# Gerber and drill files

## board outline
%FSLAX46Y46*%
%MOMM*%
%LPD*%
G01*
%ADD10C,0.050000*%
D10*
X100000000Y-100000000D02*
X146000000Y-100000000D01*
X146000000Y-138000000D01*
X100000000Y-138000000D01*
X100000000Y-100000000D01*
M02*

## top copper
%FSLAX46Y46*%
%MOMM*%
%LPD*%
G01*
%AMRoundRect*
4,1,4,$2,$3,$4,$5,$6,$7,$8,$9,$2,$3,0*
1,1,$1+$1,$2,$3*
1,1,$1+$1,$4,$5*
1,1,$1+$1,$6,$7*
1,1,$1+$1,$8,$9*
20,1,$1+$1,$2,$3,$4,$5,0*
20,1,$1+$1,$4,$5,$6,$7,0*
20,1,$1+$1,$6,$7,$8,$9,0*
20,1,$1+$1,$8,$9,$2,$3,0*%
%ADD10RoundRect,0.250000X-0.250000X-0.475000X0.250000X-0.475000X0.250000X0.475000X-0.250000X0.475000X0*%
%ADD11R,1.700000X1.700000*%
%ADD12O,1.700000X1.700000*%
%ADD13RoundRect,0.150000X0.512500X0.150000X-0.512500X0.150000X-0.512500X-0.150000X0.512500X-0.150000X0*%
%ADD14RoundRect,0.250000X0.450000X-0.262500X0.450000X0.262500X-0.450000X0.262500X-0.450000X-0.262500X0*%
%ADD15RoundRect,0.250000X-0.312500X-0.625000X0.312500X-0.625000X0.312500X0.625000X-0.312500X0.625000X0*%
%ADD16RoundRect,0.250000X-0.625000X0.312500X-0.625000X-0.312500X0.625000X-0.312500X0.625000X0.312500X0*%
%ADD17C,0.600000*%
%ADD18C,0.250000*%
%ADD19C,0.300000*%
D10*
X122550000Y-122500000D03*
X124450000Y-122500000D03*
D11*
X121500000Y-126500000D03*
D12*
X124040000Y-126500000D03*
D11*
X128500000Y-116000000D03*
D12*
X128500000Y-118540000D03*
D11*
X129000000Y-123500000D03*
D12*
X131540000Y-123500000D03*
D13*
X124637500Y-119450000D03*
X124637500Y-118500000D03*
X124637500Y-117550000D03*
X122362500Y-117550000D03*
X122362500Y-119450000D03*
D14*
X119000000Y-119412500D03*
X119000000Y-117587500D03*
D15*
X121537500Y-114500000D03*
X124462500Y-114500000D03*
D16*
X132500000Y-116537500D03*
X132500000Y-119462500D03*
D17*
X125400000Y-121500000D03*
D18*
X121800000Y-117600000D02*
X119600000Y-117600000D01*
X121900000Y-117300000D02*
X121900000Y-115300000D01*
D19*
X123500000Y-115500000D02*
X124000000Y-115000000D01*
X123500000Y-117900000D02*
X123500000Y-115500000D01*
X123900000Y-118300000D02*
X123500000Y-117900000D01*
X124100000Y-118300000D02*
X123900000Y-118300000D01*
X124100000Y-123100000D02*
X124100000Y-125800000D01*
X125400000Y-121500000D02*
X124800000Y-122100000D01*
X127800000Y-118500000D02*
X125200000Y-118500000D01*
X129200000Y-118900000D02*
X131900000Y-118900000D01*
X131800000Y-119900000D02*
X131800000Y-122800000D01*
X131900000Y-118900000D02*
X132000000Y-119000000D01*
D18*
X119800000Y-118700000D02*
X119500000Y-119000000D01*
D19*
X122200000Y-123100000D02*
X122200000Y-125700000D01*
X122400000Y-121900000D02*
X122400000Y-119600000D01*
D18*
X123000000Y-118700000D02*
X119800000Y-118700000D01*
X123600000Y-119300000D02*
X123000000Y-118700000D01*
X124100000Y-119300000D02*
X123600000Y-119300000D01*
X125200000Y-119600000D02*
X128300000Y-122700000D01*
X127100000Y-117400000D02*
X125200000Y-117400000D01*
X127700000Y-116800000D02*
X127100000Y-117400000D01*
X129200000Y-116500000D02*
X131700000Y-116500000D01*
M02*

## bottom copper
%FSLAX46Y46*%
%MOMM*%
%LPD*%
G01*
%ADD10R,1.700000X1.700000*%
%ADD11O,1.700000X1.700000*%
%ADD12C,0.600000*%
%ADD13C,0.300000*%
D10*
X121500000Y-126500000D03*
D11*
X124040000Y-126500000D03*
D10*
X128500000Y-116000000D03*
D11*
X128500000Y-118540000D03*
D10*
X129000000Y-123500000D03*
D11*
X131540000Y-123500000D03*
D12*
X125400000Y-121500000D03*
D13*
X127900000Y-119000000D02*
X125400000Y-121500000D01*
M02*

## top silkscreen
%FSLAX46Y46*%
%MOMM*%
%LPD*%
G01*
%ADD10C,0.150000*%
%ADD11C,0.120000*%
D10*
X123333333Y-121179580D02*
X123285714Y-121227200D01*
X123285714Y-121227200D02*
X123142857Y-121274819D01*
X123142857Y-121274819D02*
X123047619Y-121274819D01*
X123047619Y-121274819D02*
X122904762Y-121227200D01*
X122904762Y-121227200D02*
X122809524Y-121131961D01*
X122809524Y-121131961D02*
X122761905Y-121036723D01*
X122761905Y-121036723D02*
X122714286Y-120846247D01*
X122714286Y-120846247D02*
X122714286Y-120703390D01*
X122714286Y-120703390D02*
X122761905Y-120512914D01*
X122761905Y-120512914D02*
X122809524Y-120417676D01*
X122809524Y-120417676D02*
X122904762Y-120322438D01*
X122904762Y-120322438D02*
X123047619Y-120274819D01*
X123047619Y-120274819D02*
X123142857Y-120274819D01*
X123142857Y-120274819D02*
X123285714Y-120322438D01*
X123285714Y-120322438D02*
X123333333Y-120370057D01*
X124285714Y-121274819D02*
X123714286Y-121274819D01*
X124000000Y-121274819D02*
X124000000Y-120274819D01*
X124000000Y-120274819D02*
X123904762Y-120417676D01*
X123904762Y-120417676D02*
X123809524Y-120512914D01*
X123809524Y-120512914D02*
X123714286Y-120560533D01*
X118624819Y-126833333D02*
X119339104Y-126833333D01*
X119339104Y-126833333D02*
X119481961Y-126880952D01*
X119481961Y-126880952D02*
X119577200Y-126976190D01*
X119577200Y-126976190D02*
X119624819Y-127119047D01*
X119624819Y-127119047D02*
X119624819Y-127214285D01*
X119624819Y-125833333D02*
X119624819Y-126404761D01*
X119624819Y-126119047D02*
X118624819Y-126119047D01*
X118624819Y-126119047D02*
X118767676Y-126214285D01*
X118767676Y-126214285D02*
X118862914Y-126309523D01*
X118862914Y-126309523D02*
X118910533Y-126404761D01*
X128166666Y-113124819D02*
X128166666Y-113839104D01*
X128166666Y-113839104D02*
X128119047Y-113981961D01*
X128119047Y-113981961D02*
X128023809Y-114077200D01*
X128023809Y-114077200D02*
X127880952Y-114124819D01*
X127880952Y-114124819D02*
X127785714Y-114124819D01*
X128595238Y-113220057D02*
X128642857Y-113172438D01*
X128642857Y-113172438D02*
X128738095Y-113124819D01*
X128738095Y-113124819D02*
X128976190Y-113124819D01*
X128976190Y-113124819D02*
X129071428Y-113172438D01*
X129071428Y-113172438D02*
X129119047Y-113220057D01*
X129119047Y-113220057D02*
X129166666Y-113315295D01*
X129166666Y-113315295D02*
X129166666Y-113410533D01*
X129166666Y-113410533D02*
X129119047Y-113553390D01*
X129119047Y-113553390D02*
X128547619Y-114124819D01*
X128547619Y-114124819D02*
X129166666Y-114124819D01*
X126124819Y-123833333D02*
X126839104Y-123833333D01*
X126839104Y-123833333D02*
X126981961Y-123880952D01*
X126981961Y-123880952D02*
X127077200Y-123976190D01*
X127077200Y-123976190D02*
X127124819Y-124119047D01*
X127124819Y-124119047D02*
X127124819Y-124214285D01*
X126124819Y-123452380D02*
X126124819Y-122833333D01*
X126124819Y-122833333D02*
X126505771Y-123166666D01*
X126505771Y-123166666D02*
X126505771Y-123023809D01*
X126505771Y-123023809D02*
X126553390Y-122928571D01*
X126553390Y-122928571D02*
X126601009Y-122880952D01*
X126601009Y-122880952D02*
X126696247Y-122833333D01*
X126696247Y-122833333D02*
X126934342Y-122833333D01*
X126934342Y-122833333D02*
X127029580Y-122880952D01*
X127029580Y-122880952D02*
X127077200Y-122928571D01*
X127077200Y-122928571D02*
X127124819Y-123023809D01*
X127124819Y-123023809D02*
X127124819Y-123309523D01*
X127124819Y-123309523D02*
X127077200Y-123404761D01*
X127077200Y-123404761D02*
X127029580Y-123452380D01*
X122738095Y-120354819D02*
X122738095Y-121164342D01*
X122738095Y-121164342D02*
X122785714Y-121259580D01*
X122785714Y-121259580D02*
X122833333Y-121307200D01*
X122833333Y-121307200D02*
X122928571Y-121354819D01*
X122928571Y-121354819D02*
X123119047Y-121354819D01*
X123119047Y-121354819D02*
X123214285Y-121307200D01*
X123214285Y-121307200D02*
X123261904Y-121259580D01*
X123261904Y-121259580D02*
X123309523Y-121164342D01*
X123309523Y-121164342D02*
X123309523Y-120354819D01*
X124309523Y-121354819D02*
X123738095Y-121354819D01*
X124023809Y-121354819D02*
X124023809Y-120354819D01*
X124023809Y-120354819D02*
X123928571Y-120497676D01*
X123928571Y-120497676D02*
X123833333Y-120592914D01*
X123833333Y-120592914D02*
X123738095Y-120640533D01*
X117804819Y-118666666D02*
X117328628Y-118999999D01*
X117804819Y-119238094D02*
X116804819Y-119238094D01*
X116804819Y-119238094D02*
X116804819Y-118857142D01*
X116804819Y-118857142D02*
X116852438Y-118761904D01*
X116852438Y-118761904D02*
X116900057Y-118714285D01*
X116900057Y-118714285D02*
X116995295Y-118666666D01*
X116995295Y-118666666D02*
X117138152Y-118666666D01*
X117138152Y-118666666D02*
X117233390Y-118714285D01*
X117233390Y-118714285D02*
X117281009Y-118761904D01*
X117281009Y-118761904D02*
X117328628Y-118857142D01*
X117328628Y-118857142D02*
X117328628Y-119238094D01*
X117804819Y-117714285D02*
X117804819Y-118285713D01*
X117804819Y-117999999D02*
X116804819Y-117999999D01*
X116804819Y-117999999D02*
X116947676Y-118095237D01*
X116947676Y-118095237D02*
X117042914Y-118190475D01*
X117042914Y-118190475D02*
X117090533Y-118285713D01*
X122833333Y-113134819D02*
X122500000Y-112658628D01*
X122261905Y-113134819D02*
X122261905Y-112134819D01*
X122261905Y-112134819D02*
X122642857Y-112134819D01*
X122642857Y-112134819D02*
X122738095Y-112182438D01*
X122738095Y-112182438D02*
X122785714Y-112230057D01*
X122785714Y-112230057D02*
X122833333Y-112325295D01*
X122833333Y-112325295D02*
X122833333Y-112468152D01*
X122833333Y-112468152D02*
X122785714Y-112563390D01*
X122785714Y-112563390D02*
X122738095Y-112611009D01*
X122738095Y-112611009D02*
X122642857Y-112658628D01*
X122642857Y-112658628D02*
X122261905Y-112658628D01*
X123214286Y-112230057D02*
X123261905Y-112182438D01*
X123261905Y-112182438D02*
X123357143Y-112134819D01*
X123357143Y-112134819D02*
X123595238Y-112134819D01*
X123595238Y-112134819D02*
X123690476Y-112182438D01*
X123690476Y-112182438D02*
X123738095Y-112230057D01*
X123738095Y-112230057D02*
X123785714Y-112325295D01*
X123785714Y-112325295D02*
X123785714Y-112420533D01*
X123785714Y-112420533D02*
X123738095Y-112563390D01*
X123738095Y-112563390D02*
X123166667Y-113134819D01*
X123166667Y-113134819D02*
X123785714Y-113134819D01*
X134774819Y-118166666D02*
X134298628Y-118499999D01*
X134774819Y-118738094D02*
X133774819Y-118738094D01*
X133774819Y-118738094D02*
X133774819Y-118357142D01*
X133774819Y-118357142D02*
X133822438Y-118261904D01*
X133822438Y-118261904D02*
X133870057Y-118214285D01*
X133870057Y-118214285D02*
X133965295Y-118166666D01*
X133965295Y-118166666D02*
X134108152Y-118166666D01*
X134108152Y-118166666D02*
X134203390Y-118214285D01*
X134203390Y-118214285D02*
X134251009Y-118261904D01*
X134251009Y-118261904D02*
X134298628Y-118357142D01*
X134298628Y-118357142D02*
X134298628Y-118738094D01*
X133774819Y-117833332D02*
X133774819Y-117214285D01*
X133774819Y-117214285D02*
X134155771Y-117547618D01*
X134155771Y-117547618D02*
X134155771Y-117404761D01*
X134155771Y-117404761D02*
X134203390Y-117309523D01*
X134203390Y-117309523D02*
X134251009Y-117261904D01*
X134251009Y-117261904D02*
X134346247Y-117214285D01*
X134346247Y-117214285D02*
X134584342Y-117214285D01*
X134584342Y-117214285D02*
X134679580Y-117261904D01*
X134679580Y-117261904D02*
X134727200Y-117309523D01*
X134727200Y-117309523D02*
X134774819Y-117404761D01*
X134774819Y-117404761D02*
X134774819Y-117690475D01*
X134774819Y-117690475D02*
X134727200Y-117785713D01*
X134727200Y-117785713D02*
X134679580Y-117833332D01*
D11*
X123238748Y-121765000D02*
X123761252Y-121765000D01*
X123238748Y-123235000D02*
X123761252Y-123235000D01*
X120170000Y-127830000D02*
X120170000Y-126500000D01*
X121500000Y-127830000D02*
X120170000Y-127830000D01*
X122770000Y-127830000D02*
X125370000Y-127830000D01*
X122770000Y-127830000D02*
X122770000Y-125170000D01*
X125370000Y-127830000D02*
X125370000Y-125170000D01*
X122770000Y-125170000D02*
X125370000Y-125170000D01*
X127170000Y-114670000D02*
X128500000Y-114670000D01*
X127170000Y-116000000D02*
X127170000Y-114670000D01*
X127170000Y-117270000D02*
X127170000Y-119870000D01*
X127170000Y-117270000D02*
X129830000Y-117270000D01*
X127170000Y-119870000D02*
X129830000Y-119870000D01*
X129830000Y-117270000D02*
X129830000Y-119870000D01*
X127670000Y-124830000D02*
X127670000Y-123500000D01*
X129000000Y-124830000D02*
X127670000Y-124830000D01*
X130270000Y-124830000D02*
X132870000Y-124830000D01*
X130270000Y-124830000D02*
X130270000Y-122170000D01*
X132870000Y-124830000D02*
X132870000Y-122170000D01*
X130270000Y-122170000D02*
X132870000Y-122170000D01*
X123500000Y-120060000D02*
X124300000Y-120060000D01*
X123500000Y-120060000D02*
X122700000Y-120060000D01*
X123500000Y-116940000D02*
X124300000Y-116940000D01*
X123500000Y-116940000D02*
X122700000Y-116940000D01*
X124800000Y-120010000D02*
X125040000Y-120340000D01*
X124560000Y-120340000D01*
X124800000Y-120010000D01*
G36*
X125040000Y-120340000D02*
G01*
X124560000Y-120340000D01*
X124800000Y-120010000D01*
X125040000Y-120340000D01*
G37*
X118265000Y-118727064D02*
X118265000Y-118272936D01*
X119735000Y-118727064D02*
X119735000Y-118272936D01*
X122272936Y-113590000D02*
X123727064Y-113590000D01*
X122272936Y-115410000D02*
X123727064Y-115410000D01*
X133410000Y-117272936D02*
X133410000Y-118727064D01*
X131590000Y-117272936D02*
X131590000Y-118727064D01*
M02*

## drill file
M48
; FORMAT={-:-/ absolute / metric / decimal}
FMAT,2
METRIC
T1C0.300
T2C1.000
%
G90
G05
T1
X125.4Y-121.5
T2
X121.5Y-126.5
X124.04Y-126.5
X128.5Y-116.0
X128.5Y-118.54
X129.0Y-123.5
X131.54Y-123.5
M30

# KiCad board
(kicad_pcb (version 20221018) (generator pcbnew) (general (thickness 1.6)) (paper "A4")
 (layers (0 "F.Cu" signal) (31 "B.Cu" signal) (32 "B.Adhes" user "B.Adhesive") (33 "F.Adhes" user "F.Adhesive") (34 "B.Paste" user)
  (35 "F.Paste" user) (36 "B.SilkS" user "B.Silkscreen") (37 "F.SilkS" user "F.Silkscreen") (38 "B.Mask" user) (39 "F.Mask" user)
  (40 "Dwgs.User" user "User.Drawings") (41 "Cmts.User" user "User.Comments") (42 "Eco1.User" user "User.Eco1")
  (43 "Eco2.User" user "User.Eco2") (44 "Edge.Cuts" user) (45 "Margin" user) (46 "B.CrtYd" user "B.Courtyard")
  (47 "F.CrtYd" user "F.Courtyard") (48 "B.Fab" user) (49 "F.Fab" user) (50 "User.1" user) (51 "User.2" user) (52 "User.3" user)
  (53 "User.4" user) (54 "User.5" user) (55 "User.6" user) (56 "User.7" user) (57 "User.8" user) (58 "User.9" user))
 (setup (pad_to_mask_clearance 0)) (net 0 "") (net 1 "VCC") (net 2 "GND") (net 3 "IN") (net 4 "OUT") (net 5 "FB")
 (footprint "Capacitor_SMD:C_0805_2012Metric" (layer "F.Cu") (at 123.5 122.5)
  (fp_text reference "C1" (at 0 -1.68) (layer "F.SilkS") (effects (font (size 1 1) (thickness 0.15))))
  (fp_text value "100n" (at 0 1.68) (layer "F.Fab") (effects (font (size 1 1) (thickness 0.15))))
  (fp_line (start -0.261252 -0.735) (end 0.261252 -0.735) (stroke (width 0.12) (type solid)) (layer "F.SilkS"))
  (fp_line (start -0.261252 0.735) (end 0.261252 0.735) (stroke (width 0.12) (type solid)) (layer "F.SilkS"))
  (pad "1" smd roundrect (at -0.95 0) (size 1 1.45) (layers "F.Cu" "F.Paste" "F.Mask") (roundrect_rratio 0.25) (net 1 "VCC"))
  (pad "2" smd roundrect (at 0.95 0) (size 1 1.45) (layers "F.Cu" "F.Paste" "F.Mask") (roundrect_rratio 0.25) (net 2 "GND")))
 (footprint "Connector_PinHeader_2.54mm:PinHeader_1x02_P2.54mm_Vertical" (layer "F.Cu") (at 121.5 126.5 90)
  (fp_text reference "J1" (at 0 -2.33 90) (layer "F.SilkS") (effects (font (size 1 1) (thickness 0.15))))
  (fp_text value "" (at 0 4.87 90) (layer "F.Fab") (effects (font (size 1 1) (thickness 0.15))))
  (fp_line (start -1.33 -1.33) (end 0 -1.33) (stroke (width 0.12) (type solid)) (layer "F.SilkS"))
  (fp_line (start -1.33 0) (end -1.33 -1.33) (stroke (width 0.12) (type solid)) (layer "F.SilkS"))
  (fp_line (start -1.33 1.27) (end -1.33 3.87) (stroke (width 0.12) (type solid)) (layer "F.SilkS"))
  (fp_line (start -1.33 1.27) (end 1.33 1.27) (stroke (width 0.12) (type solid)) (layer "F.SilkS"))
  (fp_line (start -1.33 3.87) (end 1.33 3.87) (stroke (width 0.12) (type solid)) (layer "F.SilkS"))
  (fp_line (start 1.33 1.27) (end 1.33 3.87) (stroke (width 0.12) (type solid)) (layer "F.SilkS"))
  (pad "1" thru_hole rect (at 0 0 90) (size 1.7 1.7) (drill 1) (layers "*.Cu" "*.Mask") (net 1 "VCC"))
  (pad "2" thru_hole oval (at 0 2.54 90) (size 1.7 1.7) (drill 1) (layers "*.Cu" "*.Mask") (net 2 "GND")))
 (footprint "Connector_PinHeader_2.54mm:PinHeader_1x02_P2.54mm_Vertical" (layer "F.Cu") (at 128.5 116)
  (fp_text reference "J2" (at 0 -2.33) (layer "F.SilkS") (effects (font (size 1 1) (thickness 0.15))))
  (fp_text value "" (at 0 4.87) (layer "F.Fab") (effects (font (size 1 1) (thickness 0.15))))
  (fp_line (start -1.33 -1.33) (end 0 -1.33) (stroke (width 0.12) (type solid)) (layer "F.SilkS"))
  (fp_line (start -1.33 0) (end -1.33 -1.33) (stroke (width 0.12) (type solid)) (layer "F.SilkS"))
  (fp_line (start -1.33 1.27) (end -1.33 3.87) (stroke (width 0.12) (type solid)) (layer "F.SilkS"))
  (fp_line (start -1.33 1.27) (end 1.33 1.27) (stroke (width 0.12) (type solid)) (layer "F.SilkS"))
  (fp_line (start -1.33 3.87) (end 1.33 3.87) (stroke (width 0.12) (type solid)) (layer "F.SilkS"))
  (fp_line (start 1.33 1.27) (end 1.33 3.87) (stroke (width 0.12) (type solid)) (layer "F.SilkS"))
  (pad "1" thru_hole rect (at 0 0) (size 1.7 1.7) (drill 1) (layers "*.Cu" "*.Mask") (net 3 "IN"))
  (pad "2" thru_hole oval (at 0 2.54) (size 1.7 1.7) (drill 1) (layers "*.Cu" "*.Mask") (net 2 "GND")))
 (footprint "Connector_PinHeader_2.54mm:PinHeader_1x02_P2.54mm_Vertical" (layer "F.Cu") (at 129 123.5 90)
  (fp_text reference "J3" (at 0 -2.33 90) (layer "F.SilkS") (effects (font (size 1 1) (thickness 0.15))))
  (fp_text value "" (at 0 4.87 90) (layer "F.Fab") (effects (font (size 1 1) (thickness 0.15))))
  (fp_line (start -1.33 -1.33) (end 0 -1.33) (stroke (width 0.12) (type solid)) (layer "F.SilkS"))
  (fp_line (start -1.33 0) (end -1.33 -1.33) (stroke (width 0.12) (type solid)) (layer "F.SilkS"))
  (fp_line (start -1.33 1.27) (end -1.33 3.87) (stroke (width 0.12) (type solid)) (layer "F.SilkS"))
  (fp_line (start -1.33 1.27) (end 1.33 1.27) (stroke (width 0.12) (type solid)) (layer "F.SilkS"))
  (fp_line (start -1.33 3.87) (end 1.33 3.87) (stroke (width 0.12) (type solid)) (layer "F.SilkS"))
  (fp_line (start 1.33 1.27) (end 1.33 3.87) (stroke (width 0.12) (type solid)) (layer "F.SilkS"))
  (pad "1" thru_hole rect (at 0 0 90) (size 1.7 1.7) (drill 1) (layers "*.Cu" "*.Mask") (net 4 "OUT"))
  (pad "2" thru_hole oval (at 0 2.54 90) (size 1.7 1.7) (drill 1) (layers "*.Cu" "*.Mask") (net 2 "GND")))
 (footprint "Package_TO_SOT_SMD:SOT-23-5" (layer "F.Cu") (at 123.5 118.5 180)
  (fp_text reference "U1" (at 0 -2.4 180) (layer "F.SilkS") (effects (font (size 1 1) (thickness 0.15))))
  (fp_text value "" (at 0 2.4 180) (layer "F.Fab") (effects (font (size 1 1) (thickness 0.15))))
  (fp_line (start 0 -1.56) (end -0.8 -1.56) (stroke (width 0.12) (type solid)) (layer "F.SilkS"))
  (fp_line (start 0 -1.56) (end 0.8 -1.56) (stroke (width 0.12) (type solid)) (layer "F.SilkS"))
  (fp_line (start 0 1.56) (end -0.8 1.56) (stroke (width 0.12) (type solid)) (layer "F.SilkS"))
  (fp_line (start 0 1.56) (end 0.8 1.56) (stroke (width 0.12) (type solid)) (layer "F.SilkS"))
  (fp_poly
   (pts (xy -1.3 -1.51) (xy -1.54 -1.84) (xy -1.06 -1.84) (xy -1.3 -1.51)) (stroke (width 0.12) (type solid)) (fill solid) (layer "F.SilkS"))
  (pad "1" smd roundrect (at -1.1375 -0.95 180) (size 1.325 0.6) (layers "F.Cu" "F.Paste" "F.Mask") (roundrect_rratio 0.25) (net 4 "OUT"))
  (pad "2" smd roundrect (at -1.1375 0 180) (size 1.325 0.6) (layers "F.Cu" "F.Paste" "F.Mask") (roundrect_rratio 0.25) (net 2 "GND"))
  (pad "3" smd roundrect (at -1.1375 0.95 180) (size 1.325 0.6) (layers "F.Cu" "F.Paste" "F.Mask") (roundrect_rratio 0.25) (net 3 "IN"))
  (pad "4" smd roundrect (at 1.1375 0.95 180) (size 1.325 0.6) (layers "F.Cu" "F.Paste" "F.Mask") (roundrect_rratio 0.25) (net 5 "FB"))
  (pad "5" smd roundrect (at 1.1375 -0.95 180) (size 1.325 0.6) (layers "F.Cu" "F.Paste" "F.Mask") (roundrect_rratio 0.25) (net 1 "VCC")))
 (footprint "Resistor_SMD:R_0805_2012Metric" (layer "F.Cu") (at 119 118.5 90)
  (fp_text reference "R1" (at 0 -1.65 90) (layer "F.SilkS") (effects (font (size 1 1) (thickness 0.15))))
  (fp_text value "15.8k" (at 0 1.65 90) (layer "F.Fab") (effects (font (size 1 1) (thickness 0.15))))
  (fp_line (start -0.227064 -0.735) (end 0.227064 -0.735) (stroke (width 0.12) (type solid)) (layer "F.SilkS"))
  (fp_line (start -0.227064 0.735) (end 0.227064 0.735) (stroke (width 0.12) (type solid)) (layer "F.SilkS"))
  (pad "1" smd roundrect (at -0.9125 0 90) (size 1.025 1.4) (layers "F.Cu" "F.Paste" "F.Mask") (roundrect_rratio 0.243902) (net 4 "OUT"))
  (pad "2" smd roundrect (at 0.9125 0 90) (size 1.025 1.4) (layers "F.Cu" "F.Paste" "F.Mask") (roundrect_rratio 0.243902) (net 5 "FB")))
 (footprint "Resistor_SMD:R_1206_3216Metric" (layer "F.Cu") (at 123 114.5)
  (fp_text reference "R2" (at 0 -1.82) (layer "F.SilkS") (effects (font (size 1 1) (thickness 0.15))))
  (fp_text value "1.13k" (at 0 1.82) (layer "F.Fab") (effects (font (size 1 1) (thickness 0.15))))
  (fp_line (start -0.727064 -0.91) (end 0.727064 -0.91) (stroke (width 0.12) (type solid)) (layer "F.SilkS"))
  (fp_line (start -0.727064 0.91) (end 0.727064 0.91) (stroke (width 0.12) (type solid)) (layer "F.SilkS"))
  (pad "1" smd roundrect (at -1.4625 0) (size 1.125 1.75) (layers "F.Cu" "F.Paste" "F.Mask") (roundrect_rratio 0.222222) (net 5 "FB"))
  (pad "2" smd roundrect (at 1.4625 0) (size 1.125 1.75) (layers "F.Cu" "F.Paste" "F.Mask") (roundrect_rratio 0.222222) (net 2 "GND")))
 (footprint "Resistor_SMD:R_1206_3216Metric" (layer "F.Cu") (at 132.5 118 -90)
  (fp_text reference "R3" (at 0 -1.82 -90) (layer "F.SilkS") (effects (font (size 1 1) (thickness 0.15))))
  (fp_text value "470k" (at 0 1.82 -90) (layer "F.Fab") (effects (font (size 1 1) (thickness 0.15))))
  (fp_line (start -0.727064 -0.91) (end 0.727064 -0.91) (stroke (width 0.12) (type solid)) (layer "F.SilkS"))
  (fp_line (start -0.727064 0.91) (end 0.727064 0.91) (stroke (width 0.12) (type solid)) (layer "F.SilkS"))
  (pad "1" smd roundrect (at -1.4625 0 270) (size 1.125 1.75) (layers "F.Cu" "F.Paste" "F.Mask") (roundrect_rratio 0.222222) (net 3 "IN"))
  (pad "2" smd roundrect (at 1.4625 0 270) (size 1.125 1.75) (layers "F.Cu" "F.Paste" "F.Mask") (roundrect_rratio 0.222222) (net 2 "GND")))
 (gr_rect (start 100 100) (end 146 138) (stroke (width 0.05) (type default)) (fill none) (layer "Edge.Cuts"))
 (segment (start 121.8 117.6) (end 119.6 117.6) (width 0.25) (layer "F.Cu") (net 5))
 (segment (start 121.9 117.3) (end 121.9 115.3) (width 0.25) (layer "F.Cu") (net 5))
 (segment (start 123.5 115.5) (end 124 115) (width 0.3) (layer "F.Cu") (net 2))
 (segment (start 123.5 117.9) (end 123.5 115.5) (width 0.3) (layer "F.Cu") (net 2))
 (segment (start 123.9 118.3) (end 123.5 117.9) (width 0.3) (layer "F.Cu") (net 2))
 (segment (start 124.1 118.3) (end 123.9 118.3) (width 0.3) (layer "F.Cu") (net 2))
 (segment (start 124.1 123.1) (end 124.1 125.8) (width 0.3) (layer "F.Cu") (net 2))
 (segment (start 125.4 121.5) (end 124.8 122.1) (width 0.3) (layer "F.Cu") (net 2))
 (segment (start 127.8 118.5) (end 125.2 118.5) (width 0.3) (layer "F.Cu") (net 2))
 (segment (start 129.2 118.9) (end 131.9 118.9) (width 0.3) (layer "F.Cu") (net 2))
 (segment (start 131.8 119.9) (end 131.8 122.8) (width 0.3) (layer "F.Cu") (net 2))
 (segment (start 131.9 118.9) (end 132 119) (width 0.3) (layer "F.Cu") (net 2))
 (via (at 125.4 121.5) (size 0.6) (drill 0.3) (layers "F.Cu" "B.Cu") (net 2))
 (segment (start 119.8 118.7) (end 119.5 119) (width 0.25) (layer "F.Cu") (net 4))
 (segment (start 122.2 123.1) (end 122.2 125.7) (width 0.3) (layer "F.Cu") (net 1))
 (segment (start 122.4 121.9) (end 122.4 119.6) (width 0.3) (layer "F.Cu") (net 1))
 (segment (start 123 118.7) (end 119.8 118.7) (width 0.25) (layer "F.Cu") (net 4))
 (segment (start 123.6 119.3) (end 123 118.7) (width 0.25) (layer "F.Cu") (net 4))
 (segment (start 124.1 119.3) (end 123.6 119.3) (width 0.25) (layer "F.Cu") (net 4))
 (segment (start 125.2 119.6) (end 128.3 122.7) (width 0.25) (layer "F.Cu") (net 4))
 (segment (start 127.1 117.4) (end 125.2 117.4) (width 0.25) (layer "F.Cu") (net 3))
 (segment (start 127.7 116.8) (end 127.1 117.4) (width 0.25) (layer "F.Cu") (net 3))
 (segment (start 127.9 119) (end 125.4 121.5) (width 0.3) (layer "B.Cu") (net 2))
 (segment (start 129.2 116.5) (end 131.7 116.5) (width 0.25) (layer "F.Cu") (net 3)))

